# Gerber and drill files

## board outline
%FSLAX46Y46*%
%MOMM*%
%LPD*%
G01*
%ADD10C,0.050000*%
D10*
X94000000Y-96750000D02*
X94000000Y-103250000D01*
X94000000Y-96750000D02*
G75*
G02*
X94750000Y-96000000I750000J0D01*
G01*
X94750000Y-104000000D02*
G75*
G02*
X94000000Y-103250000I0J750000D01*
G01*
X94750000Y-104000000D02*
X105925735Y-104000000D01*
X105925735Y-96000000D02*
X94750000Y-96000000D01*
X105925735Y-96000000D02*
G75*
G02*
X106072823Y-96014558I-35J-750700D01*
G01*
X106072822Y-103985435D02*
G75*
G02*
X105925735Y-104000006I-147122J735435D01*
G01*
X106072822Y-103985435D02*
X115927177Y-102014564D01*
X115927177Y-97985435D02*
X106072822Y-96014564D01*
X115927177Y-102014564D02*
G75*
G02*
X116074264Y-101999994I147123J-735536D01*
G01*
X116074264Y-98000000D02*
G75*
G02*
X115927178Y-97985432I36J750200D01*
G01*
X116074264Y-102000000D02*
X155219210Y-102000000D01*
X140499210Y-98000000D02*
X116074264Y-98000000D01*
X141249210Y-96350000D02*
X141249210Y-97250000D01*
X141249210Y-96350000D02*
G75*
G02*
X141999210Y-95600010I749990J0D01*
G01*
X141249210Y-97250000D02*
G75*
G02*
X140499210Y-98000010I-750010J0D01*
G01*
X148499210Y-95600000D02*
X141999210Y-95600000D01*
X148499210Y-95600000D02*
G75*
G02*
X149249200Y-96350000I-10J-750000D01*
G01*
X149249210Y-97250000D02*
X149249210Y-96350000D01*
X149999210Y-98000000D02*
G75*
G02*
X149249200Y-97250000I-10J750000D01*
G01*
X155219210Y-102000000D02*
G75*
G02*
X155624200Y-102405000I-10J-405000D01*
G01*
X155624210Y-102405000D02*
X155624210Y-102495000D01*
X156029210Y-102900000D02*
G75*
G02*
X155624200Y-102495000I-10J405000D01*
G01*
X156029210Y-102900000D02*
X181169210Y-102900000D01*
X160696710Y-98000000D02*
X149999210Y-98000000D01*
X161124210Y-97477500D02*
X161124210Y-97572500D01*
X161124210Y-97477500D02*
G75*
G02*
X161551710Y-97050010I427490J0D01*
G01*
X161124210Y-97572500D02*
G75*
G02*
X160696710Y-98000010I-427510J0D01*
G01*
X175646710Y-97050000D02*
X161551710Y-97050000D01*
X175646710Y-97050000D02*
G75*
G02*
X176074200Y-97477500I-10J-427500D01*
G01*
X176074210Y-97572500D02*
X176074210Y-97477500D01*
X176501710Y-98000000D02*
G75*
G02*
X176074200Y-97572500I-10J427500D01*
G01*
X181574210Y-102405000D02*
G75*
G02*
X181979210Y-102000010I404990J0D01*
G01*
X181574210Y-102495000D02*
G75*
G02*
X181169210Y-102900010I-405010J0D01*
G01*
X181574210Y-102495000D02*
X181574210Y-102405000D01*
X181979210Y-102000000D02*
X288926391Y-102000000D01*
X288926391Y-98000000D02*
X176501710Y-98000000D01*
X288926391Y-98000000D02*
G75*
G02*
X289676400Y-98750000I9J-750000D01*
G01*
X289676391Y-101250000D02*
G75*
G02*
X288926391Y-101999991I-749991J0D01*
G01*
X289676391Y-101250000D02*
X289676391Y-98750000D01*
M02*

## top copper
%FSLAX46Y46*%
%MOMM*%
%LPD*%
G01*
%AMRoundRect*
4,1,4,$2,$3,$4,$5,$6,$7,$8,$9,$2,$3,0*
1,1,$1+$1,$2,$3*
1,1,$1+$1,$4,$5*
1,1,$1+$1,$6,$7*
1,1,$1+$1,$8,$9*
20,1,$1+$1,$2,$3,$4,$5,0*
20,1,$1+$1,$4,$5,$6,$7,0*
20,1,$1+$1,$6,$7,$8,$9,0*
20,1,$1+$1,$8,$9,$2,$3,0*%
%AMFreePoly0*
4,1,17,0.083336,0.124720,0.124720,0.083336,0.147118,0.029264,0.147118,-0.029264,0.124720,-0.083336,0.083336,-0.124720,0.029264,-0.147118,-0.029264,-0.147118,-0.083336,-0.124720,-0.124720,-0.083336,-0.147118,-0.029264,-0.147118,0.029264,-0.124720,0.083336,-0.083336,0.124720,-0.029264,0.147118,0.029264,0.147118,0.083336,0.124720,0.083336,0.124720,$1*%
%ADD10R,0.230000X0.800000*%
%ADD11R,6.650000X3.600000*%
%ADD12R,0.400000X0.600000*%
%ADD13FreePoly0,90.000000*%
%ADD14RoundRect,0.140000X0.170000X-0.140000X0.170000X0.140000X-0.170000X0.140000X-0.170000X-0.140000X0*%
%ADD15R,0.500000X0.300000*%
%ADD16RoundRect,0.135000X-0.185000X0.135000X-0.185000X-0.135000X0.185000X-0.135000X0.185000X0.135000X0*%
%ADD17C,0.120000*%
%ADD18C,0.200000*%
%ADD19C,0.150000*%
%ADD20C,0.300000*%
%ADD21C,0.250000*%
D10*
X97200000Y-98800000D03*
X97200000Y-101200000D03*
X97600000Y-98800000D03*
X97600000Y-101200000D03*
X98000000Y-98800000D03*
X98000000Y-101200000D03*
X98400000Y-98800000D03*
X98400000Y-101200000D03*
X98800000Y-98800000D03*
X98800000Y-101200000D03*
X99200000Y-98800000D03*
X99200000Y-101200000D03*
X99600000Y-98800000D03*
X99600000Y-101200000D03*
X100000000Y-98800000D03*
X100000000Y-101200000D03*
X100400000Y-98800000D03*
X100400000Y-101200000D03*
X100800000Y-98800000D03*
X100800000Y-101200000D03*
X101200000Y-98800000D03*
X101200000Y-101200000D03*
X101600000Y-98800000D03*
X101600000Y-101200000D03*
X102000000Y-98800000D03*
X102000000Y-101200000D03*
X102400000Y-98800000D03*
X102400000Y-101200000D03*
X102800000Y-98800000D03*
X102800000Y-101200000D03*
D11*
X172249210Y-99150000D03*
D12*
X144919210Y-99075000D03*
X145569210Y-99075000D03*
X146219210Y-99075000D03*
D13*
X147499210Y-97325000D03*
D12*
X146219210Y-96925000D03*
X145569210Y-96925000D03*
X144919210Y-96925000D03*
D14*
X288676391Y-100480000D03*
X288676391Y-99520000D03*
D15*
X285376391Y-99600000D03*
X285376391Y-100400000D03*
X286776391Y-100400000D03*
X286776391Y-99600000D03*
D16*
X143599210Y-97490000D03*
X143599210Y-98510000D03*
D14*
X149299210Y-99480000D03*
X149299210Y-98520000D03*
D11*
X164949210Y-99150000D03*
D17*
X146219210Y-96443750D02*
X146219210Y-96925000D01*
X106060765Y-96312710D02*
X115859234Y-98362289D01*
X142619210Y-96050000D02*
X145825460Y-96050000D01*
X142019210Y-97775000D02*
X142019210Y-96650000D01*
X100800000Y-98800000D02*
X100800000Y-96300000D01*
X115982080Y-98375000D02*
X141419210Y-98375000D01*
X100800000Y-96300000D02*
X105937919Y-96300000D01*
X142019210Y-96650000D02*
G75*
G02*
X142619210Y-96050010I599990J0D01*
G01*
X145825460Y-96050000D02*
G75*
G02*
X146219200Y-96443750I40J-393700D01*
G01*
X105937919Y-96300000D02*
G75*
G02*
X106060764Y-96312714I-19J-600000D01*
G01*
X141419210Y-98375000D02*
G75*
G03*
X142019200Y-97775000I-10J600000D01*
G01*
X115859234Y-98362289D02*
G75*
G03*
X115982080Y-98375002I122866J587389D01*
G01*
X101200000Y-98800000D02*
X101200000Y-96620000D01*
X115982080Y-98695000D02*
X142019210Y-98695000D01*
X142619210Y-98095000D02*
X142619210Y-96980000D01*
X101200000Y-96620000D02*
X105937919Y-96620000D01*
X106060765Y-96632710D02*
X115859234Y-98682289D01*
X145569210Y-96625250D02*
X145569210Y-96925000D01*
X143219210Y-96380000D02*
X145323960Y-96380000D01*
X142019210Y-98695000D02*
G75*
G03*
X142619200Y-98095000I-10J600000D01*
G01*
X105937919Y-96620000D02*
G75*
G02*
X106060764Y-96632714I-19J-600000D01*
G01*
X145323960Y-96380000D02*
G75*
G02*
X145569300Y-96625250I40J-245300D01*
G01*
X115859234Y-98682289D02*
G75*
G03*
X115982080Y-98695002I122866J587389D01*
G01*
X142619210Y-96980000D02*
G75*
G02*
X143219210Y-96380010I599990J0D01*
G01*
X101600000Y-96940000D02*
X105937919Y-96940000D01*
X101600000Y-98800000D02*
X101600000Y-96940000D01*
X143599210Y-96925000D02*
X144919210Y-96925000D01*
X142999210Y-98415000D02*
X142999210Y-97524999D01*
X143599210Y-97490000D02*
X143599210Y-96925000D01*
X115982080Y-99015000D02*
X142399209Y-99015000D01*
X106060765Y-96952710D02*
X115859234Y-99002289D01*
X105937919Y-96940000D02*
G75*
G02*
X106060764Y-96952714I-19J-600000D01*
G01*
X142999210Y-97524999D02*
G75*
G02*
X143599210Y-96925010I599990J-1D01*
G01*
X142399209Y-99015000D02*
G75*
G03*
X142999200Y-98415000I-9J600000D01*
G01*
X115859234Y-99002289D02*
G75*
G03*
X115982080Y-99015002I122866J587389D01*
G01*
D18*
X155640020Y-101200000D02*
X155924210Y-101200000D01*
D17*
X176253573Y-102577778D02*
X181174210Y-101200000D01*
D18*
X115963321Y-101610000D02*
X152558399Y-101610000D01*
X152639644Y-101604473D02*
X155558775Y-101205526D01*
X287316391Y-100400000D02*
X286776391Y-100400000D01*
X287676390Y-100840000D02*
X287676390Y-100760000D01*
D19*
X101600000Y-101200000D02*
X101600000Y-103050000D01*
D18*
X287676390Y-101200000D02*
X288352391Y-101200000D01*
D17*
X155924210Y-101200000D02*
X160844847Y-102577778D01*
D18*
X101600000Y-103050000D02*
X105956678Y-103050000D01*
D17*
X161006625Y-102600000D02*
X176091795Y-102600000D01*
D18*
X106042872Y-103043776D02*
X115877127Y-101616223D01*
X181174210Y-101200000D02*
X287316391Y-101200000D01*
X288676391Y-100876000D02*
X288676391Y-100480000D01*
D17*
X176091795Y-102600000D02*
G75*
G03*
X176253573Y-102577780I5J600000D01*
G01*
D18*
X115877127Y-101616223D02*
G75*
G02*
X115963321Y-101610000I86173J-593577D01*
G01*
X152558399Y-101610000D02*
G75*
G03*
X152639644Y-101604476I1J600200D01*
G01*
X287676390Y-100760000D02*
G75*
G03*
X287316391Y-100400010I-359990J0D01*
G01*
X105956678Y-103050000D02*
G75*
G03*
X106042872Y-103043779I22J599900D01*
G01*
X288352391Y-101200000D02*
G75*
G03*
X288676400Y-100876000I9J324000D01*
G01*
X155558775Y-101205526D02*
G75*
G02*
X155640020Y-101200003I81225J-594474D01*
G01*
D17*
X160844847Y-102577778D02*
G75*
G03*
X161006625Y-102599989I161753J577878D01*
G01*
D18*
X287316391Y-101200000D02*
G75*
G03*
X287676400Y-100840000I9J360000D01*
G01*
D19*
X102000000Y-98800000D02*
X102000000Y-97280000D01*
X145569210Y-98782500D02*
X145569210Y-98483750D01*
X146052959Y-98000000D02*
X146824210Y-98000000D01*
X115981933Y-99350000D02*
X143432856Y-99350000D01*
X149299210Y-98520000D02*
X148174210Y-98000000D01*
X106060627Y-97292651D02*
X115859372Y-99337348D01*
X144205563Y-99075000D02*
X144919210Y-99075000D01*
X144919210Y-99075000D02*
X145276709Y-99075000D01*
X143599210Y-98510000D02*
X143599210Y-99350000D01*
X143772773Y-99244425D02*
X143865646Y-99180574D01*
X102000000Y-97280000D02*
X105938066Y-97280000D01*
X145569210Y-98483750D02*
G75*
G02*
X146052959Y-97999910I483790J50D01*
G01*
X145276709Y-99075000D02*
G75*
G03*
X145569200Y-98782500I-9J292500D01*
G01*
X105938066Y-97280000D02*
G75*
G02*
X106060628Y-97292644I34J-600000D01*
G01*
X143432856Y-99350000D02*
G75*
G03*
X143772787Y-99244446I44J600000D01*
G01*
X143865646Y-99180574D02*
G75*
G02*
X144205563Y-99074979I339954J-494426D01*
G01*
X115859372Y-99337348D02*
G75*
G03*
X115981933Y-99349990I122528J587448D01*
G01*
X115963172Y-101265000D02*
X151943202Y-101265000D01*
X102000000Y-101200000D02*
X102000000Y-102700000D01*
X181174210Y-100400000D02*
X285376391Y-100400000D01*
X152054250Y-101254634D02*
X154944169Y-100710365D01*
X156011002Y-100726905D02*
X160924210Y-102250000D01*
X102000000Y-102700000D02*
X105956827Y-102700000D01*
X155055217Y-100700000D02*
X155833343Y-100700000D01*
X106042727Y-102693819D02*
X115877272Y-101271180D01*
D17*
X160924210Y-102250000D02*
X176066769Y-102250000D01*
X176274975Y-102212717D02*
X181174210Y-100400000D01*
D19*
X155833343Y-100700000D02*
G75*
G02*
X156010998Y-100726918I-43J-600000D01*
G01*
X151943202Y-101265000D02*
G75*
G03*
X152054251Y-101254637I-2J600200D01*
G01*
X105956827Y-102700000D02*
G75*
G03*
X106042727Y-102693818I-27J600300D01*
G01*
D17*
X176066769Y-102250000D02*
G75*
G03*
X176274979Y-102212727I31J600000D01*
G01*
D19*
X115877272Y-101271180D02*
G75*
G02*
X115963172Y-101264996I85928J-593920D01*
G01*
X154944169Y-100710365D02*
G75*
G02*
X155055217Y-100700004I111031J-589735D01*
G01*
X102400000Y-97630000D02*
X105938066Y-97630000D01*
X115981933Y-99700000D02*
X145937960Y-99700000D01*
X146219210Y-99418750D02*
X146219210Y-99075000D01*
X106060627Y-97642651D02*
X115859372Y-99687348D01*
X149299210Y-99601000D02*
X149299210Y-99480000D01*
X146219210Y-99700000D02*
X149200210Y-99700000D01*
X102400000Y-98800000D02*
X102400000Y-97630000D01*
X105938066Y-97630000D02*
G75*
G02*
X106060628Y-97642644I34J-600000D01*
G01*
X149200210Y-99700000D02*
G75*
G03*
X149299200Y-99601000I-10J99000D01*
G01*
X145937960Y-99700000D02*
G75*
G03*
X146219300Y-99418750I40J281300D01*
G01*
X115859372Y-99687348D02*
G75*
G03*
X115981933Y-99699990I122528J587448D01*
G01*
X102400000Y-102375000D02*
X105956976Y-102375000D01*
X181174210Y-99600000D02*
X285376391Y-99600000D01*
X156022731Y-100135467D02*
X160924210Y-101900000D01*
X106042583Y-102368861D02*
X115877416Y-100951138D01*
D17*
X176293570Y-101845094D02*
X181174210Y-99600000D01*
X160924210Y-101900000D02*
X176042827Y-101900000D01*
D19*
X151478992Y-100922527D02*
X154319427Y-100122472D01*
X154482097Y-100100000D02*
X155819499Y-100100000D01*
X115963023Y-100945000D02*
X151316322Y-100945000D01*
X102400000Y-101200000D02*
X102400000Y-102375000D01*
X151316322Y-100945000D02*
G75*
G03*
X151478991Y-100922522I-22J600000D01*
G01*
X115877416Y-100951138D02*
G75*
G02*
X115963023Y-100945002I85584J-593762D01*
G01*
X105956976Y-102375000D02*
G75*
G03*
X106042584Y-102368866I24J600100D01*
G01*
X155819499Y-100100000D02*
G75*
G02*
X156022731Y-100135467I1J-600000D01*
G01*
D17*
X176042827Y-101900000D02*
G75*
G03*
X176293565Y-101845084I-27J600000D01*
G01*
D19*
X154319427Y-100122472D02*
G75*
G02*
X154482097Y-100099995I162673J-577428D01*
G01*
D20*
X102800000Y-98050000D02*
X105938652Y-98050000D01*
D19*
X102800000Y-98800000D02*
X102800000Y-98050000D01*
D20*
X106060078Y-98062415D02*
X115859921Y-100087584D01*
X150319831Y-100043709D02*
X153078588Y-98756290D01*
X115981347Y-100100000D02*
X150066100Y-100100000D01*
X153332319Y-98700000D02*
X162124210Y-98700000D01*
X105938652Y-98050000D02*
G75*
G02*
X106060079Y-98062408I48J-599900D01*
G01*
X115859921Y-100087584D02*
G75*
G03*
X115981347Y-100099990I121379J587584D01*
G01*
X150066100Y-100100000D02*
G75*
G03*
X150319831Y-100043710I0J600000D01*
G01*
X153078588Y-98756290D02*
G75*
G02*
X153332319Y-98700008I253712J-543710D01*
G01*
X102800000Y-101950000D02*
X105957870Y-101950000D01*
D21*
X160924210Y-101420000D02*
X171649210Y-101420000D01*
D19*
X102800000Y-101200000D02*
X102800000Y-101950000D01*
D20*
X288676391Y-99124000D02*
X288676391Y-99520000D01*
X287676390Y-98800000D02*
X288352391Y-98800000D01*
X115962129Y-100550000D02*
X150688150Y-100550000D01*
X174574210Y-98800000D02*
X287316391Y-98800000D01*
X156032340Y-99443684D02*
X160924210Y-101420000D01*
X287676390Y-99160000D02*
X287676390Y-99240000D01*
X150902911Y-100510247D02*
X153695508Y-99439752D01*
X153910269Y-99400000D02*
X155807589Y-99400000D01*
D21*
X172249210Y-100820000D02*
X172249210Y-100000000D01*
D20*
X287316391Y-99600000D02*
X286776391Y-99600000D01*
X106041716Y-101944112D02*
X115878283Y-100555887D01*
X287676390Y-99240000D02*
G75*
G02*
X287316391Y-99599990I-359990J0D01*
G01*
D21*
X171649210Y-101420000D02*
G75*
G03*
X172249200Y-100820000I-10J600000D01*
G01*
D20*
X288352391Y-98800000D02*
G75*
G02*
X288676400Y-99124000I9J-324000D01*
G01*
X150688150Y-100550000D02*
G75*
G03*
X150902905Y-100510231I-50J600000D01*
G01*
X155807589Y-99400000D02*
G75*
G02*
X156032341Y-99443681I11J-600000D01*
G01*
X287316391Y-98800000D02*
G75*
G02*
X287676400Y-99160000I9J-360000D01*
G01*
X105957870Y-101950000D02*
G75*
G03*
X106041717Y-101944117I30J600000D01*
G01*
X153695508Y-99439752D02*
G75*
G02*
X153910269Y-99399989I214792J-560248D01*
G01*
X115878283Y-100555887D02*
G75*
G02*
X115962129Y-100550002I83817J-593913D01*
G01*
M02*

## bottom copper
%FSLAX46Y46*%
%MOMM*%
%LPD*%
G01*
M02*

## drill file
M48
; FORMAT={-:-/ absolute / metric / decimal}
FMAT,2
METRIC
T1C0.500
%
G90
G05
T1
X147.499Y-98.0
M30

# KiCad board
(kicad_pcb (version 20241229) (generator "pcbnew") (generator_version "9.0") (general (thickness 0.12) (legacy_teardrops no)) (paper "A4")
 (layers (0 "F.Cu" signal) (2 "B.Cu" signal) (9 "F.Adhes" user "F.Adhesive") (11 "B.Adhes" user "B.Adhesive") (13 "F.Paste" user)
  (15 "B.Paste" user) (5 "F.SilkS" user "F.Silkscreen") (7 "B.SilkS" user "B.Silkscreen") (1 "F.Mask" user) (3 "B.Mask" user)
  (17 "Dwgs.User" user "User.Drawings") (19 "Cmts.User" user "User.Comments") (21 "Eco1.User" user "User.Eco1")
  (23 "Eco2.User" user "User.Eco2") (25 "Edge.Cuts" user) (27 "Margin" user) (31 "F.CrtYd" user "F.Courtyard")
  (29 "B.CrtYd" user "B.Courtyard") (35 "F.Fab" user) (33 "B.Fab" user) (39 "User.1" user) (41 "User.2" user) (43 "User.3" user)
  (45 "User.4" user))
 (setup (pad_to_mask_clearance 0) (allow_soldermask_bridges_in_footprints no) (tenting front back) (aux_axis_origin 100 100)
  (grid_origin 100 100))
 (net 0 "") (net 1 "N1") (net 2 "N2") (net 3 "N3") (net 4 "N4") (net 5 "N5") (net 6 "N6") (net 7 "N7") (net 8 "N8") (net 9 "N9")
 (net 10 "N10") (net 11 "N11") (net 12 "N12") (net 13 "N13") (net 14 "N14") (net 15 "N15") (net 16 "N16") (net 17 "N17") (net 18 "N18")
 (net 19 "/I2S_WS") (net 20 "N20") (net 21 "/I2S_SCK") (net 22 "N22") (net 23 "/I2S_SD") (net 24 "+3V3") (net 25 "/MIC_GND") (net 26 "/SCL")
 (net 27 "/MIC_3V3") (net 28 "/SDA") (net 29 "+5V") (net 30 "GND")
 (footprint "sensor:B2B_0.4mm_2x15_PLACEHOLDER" (layer "F.Cu") (at 100 100)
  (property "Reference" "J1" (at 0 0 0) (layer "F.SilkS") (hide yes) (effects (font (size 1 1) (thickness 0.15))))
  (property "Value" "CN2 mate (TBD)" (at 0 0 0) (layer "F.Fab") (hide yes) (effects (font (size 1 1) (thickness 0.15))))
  (pad "1" smd rect (at -2.8 -1.2) (size 0.23 0.8) (layers "F.Cu" "F.Mask" "F.Paste") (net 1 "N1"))
  (pad "2" smd rect (at -2.8 1.2) (size 0.23 0.8) (layers "F.Cu" "F.Mask" "F.Paste") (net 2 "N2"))
  (pad "3" smd rect (at -2.4 -1.2) (size 0.23 0.8) (layers "F.Cu" "F.Mask" "F.Paste") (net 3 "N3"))
  (pad "4" smd rect (at -2.4 1.2) (size 0.23 0.8) (layers "F.Cu" "F.Mask" "F.Paste") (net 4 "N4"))
  (pad "5" smd rect (at -2 -1.2) (size 0.23 0.8) (layers "F.Cu" "F.Mask" "F.Paste") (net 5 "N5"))
  (pad "6" smd rect (at -2 1.2) (size 0.23 0.8) (layers "F.Cu" "F.Mask" "F.Paste") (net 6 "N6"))
  (pad "7" smd rect (at -1.6 -1.2) (size 0.23 0.8) (layers "F.Cu" "F.Mask" "F.Paste") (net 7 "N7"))
  (pad "8" smd rect (at -1.6 1.2) (size 0.23 0.8) (layers "F.Cu" "F.Mask" "F.Paste") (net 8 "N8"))
  (pad "9" smd rect (at -1.2 -1.2) (size 0.23 0.8) (layers "F.Cu" "F.Mask" "F.Paste") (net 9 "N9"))
  (pad "10" smd rect (at -1.2 1.2) (size 0.23 0.8) (layers "F.Cu" "F.Mask" "F.Paste") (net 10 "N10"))
  (pad "11" smd rect (at -0.8 -1.2) (size 0.23 0.8) (layers "F.Cu" "F.Mask" "F.Paste") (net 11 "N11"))
  (pad "12" smd rect (at -0.8 1.2) (size 0.23 0.8) (layers "F.Cu" "F.Mask" "F.Paste") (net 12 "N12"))
  (pad "13" smd rect (at -0.4 -1.2) (size 0.23 0.8) (layers "F.Cu" "F.Mask" "F.Paste") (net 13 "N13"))
  (pad "14" smd rect (at -0.4 1.2) (size 0.23 0.8) (layers "F.Cu" "F.Mask" "F.Paste") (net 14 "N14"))
  (pad "15" smd rect (at 0 -1.2) (size 0.23 0.8) (layers "F.Cu" "F.Mask" "F.Paste") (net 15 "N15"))
  (pad "16" smd rect (at 0 1.2) (size 0.23 0.8) (layers "F.Cu" "F.Mask" "F.Paste") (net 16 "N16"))
  (pad "17" smd rect (at 0.4 -1.2) (size 0.23 0.8) (layers "F.Cu" "F.Mask" "F.Paste") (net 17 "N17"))
  (pad "18" smd rect (at 0.4 1.2) (size 0.23 0.8) (layers "F.Cu" "F.Mask" "F.Paste") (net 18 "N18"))
  (pad "19" smd rect (at 0.8 -1.2) (size 0.23 0.8) (layers "F.Cu" "F.Mask" "F.Paste") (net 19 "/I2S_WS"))
  (pad "20" smd rect (at 0.8 1.2) (size 0.23 0.8) (layers "F.Cu" "F.Mask" "F.Paste") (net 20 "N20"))
  (pad "21" smd rect (at 1.2 -1.2) (size 0.23 0.8) (layers "F.Cu" "F.Mask" "F.Paste") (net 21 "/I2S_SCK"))
  (pad "22" smd rect (at 1.2 1.2) (size 0.23 0.8) (layers "F.Cu" "F.Mask" "F.Paste") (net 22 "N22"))
  (pad "23" smd rect (at 1.6 -1.2) (size 0.23 0.8) (layers "F.Cu" "F.Mask" "F.Paste") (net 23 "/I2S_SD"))
  (pad "24" smd rect (at 1.6 1.2) (size 0.23 0.8) (layers "F.Cu" "F.Mask" "F.Paste") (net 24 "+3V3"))
  (pad "25" smd rect (at 2 -1.2) (size 0.23 0.8) (layers "F.Cu" "F.Mask" "F.Paste") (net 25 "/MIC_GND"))
  (pad "26" smd rect (at 2 1.2) (size 0.23 0.8) (layers "F.Cu" "F.Mask" "F.Paste") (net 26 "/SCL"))
  (pad "27" smd rect (at 2.4 -1.2) (size 0.23 0.8) (layers "F.Cu" "F.Mask" "F.Paste") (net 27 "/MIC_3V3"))
  (pad "28" smd rect (at 2.4 1.2) (size 0.23 0.8) (layers "F.Cu" "F.Mask" "F.Paste") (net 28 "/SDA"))
  (pad "29" smd rect (at 2.8 -1.2) (size 0.23 0.8) (layers "F.Cu" "F.Mask" "F.Paste") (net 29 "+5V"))
  (pad "30" smd rect (at 2.8 1.2) (size 0.23 0.8) (layers "F.Cu" "F.Mask" "F.Paste") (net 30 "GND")))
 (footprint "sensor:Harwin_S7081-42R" (layer "F.Cu") (at 172.24921 99.15)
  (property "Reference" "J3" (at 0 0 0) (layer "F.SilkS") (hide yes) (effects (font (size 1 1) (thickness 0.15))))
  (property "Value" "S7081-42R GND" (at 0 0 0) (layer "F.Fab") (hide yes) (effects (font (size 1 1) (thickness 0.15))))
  (pad "1" smd rect (at 0 0) (size 6.65 3.6) (layers "F.Cu" "F.Mask" "F.Paste") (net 30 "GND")))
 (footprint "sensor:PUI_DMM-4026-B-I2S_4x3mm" (layer "F.Cu") (at 146.49921 98 90)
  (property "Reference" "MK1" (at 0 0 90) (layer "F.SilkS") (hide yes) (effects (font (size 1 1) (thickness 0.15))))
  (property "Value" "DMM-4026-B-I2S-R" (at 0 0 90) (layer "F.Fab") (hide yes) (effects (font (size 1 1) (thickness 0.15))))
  (pad "" np_thru_hole circle (at 0 1 90) (size 0.5 0.5) (drill 0.5) (layers "*.Mask"))
  (pad "1" smd rect (at -1.075 -1.58 90) (size 0.6 0.4) (layers "F.Cu" "F.Mask" "F.Paste") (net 25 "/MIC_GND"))
  (pad "2" smd rect (at -1.075 -0.93 90) (size 0.6 0.4) (layers "F.Cu" "F.Mask" "F.Paste") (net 25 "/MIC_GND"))
  (pad "3" smd rect (at -1.075 -0.28 90) (size 0.6 0.4) (layers "F.Cu" "F.Mask" "F.Paste") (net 27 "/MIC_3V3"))
  (pad "4" smd custom (at 0.675 1 90) (size 0.3 0.3) (layers "F.Cu" "F.Mask" "F.Paste") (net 25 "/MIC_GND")
   (options (clearance outline) (anchor circle)) (primitives))
  (pad "5" smd rect (at 1.075 -0.28 90) (size 0.6 0.4) (layers "F.Cu" "F.Mask" "F.Paste") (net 19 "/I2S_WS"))
  (pad "6" smd rect (at 1.075 -0.93 90) (size 0.6 0.4) (layers "F.Cu" "F.Mask" "F.Paste") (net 21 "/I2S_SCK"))
  (pad "7" smd rect (at 1.075 -1.58 90) (size 0.6 0.4) (layers "F.Cu" "F.Mask" "F.Paste") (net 23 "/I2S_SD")))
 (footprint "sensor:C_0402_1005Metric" (layer "F.Cu") (at 288.676391 100 90)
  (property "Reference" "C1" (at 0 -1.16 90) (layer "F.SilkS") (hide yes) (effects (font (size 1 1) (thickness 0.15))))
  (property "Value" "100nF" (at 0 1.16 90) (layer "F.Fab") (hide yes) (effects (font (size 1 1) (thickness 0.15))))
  (pad "1" smd roundrect (at -0.48 0 90) (size 0.56 0.62) (layers "F.Cu" "F.Mask" "F.Paste") (roundrect_rratio 0.25) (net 24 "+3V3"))
  (pad "2" smd roundrect (at 0.48 0 90) (size 0.56 0.62) (layers "F.Cu" "F.Mask" "F.Paste") (roundrect_rratio 0.25) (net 30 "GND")))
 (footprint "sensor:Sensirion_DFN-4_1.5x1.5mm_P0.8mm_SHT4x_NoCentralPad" (layer "F.Cu") (at 286.076391 100)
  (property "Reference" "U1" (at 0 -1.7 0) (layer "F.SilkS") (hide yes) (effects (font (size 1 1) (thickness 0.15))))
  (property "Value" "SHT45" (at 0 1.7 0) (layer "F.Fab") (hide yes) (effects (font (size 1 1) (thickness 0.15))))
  (pad "1" smd rect (at -0.7 -0.4) (size 0.5 0.3) (layers "F.Cu" "F.Mask" "F.Paste") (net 28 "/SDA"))
  (pad "2" smd rect (at -0.7 0.4) (size 0.5 0.3) (layers "F.Cu" "F.Mask" "F.Paste") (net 26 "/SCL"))
  (pad "3" smd rect (at 0.7 0.4) (size 0.5 0.3) (layers "F.Cu" "F.Mask" "F.Paste") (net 24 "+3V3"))
  (pad "4" smd rect (at 0.7 -0.4) (size 0.5 0.3) (layers "F.Cu" "F.Mask" "F.Paste") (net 30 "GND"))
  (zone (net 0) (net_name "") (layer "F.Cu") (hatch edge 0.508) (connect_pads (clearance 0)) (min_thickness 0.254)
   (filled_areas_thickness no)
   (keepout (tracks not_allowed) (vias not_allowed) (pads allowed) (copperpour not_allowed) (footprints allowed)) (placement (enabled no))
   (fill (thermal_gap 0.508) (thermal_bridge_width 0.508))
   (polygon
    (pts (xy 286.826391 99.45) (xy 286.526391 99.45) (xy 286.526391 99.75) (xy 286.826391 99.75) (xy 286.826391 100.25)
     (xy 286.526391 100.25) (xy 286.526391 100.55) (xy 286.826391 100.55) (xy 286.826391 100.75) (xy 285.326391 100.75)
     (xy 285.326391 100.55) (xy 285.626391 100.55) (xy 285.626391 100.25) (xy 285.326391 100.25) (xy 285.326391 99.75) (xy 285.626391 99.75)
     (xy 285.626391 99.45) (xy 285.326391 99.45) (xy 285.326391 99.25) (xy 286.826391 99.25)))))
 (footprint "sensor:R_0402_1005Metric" (layer "F.Cu") (at 143.59921 98 -90)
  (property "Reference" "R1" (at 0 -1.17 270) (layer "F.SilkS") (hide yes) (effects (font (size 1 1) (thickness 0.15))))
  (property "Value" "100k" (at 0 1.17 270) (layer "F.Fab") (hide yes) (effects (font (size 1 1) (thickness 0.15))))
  (pad "1" smd roundrect (at -0.51 0 270) (size 0.54 0.64) (layers "F.Cu" "F.Mask" "F.Paste") (roundrect_rratio 0.25) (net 23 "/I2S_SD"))
  (pad "2" smd roundrect (at 0.51 0 270) (size 0.54 0.64) (layers "F.Cu" "F.Mask" "F.Paste") (roundrect_rratio 0.25) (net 25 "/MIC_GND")))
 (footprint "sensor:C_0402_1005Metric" (layer "F.Cu") (at 149.29921 99 90)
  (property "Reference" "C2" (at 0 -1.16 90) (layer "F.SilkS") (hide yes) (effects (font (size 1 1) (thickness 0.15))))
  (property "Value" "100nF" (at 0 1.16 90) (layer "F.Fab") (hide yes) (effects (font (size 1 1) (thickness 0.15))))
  (pad "1" smd roundrect (at -0.48 0 90) (size 0.56 0.62) (layers "F.Cu" "F.Mask" "F.Paste") (roundrect_rratio 0.25) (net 27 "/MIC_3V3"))
  (pad "2" smd roundrect (at 0.48 0 90) (size 0.56 0.62) (layers "F.Cu" "F.Mask" "F.Paste") (roundrect_rratio 0.25) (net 25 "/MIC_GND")))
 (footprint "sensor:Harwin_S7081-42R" (layer "F.Cu") (at 164.94921 99.15)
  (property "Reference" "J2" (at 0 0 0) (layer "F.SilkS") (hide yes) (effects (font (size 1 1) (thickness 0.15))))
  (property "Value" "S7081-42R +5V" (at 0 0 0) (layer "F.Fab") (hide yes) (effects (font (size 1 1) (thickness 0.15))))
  (pad "1" smd rect (at 0 0) (size 6.65 3.6) (layers "F.Cu" "F.Mask" "F.Paste") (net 29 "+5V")))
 (gr_line (start 94 96.75) (end 94 103.25) (stroke (width 0.05) (type default)) (layer "Edge.Cuts"))
 (gr_arc (start 94 96.75) (mid 94.21967 96.21967) (end 94.75 96) (stroke (width 0.05) (type default)) (layer "Edge.Cuts"))
 (gr_arc (start 94.75 104) (mid 94.21967 103.78033) (end 94 103.25) (stroke (width 0.05) (type default)) (layer "Edge.Cuts"))
 (gr_line (start 94.75 104) (end 105.925735 104) (stroke (width 0.05) (type default)) (layer "Edge.Cuts"))
 (gr_line (start 105.925735 96) (end 94.75 96) (stroke (width 0.05) (type default)) (layer "Edge.Cuts"))
 (gr_arc (start 105.925735 96) (mid 105.999638 96.003653) (end 106.072822 96.014564) (stroke (width 0.05) (type default))
  (layer "Edge.Cuts"))
 (gr_arc (start 106.072822 103.985435) (mid 105.999638 103.99635) (end 105.925735 104) (stroke (width 0.05) (type default))
  (layer "Edge.Cuts"))
 (gr_line (start 106.072822 103.985435) (end 115.927177 102.014564) (stroke (width 0.05) (type default)) (layer "Edge.Cuts"))
 (gr_line (start 115.927177 97.985435) (end 106.072822 96.014564) (stroke (width 0.05) (type default)) (layer "Edge.Cuts"))
 (gr_arc (start 115.927177 102.014564) (mid 116.000361 102.00365) (end 116.074264 102) (stroke (width 0.05) (type default))
  (layer "Edge.Cuts"))
 (gr_arc (start 116.074264 98) (mid 116.000361 97.996349) (end 115.927177 97.985435) (stroke (width 0.05) (type default))
  (layer "Edge.Cuts"))
 (gr_line (start 116.074264 102) (end 155.21921 102) (stroke (width 0.05) (type default)) (layer "Edge.Cuts"))
 (gr_line (start 140.49921 98) (end 116.074264 98) (stroke (width 0.05) (type default)) (layer "Edge.Cuts"))
 (gr_line (start 141.24921 96.35) (end 141.24921 97.25) (stroke (width 0.05) (type default)) (layer "Edge.Cuts"))
 (gr_arc (start 141.24921 96.35) (mid 141.468881 95.819673) (end 141.99921 95.6) (stroke (width 0.05) (type default)) (layer "Edge.Cuts"))
 (gr_arc (start 141.24921 97.25) (mid 141.02954 97.78033) (end 140.49921 98) (stroke (width 0.05) (type default)) (layer "Edge.Cuts"))
 (gr_line (start 148.49921 95.6) (end 141.99921 95.6) (stroke (width 0.05) (type default)) (layer "Edge.Cuts"))
 (gr_arc (start 148.49921 95.6) (mid 149.029534 95.819673) (end 149.24921 96.35) (stroke (width 0.05) (type default)) (layer "Edge.Cuts"))
 (gr_line (start 149.24921 97.25) (end 149.24921 96.35) (stroke (width 0.05) (type default)) (layer "Edge.Cuts"))
 (gr_arc (start 149.99921 98) (mid 149.46888 97.78033) (end 149.24921 97.25) (stroke (width 0.05) (type default)) (layer "Edge.Cuts"))
 (gr_arc (start 155.21921 102) (mid 155.505588 102.118621) (end 155.62421 102.405) (stroke (width 0.05) (type default)) (layer "Edge.Cuts"))
 (gr_line (start 155.62421 102.405) (end 155.62421 102.495) (stroke (width 0.05) (type default)) (layer "Edge.Cuts"))
 (gr_arc (start 156.02921 102.9) (mid 155.742825 102.781382) (end 155.62421 102.495) (stroke (width 0.05) (type default))
  (layer "Edge.Cuts"))
 (gr_line (start 156.02921 102.9) (end 181.16921 102.9) (stroke (width 0.05) (type default)) (layer "Edge.Cuts"))
 (gr_line (start 160.69671 98) (end 149.99921 98) (stroke (width 0.05) (type default)) (layer "Edge.Cuts"))
 (gr_line (start 161.12421 97.4775) (end 161.12421 97.5725) (stroke (width 0.05) (type default)) (layer "Edge.Cuts"))
 (gr_arc (start 161.12421 97.4775) (mid 161.249422 97.175215) (end 161.55171 97.05) (stroke (width 0.05) (type default)) (layer "Edge.Cuts"))
 (gr_arc (start 161.12421 97.5725) (mid 160.998998 97.874788) (end 160.69671 98) (stroke (width 0.05) (type default)) (layer "Edge.Cuts"))
 (gr_line (start 175.64671 97.05) (end 161.55171 97.05) (stroke (width 0.05) (type default)) (layer "Edge.Cuts"))
 (gr_arc (start 175.64671 97.05) (mid 175.948992 97.175215) (end 176.07421 97.4775) (stroke (width 0.05) (type default)) (layer "Edge.Cuts"))
 (gr_line (start 176.07421 97.5725) (end 176.07421 97.4775) (stroke (width 0.05) (type default)) (layer "Edge.Cuts"))
 (gr_arc (start 176.50171 98) (mid 176.199422 97.874788) (end 176.07421 97.5725) (stroke (width 0.05) (type default)) (layer "Edge.Cuts"))
 (gr_arc (start 181.57421 102.405) (mid 181.692832 102.118621) (end 181.97921 102) (stroke (width 0.05) (type default)) (layer "Edge.Cuts"))
 (gr_arc (start 181.57421 102.495) (mid 181.455589 102.781382) (end 181.16921 102.9) (stroke (width 0.05) (type default))
  (layer "Edge.Cuts"))
 (gr_line (start 181.57421 102.495) (end 181.57421 102.405) (stroke (width 0.05) (type default)) (layer "Edge.Cuts"))
 (gr_line (start 181.97921 102) (end 288.926391 102) (stroke (width 0.05) (type default)) (layer "Edge.Cuts"))
 (gr_line (start 288.926391 98) (end 176.50171 98) (stroke (width 0.05) (type default)) (layer "Edge.Cuts"))
 (gr_arc (start 288.926391 98) (mid 289.456727 98.219667) (end 289.676391 98.75) (stroke (width 0.05) (type default)) (layer "Edge.Cuts"))
 (gr_arc (start 289.676391 101.25) (mid 289.456721 101.780327) (end 288.926391 102) (stroke (width 0.05) (type default)) (layer "Edge.Cuts"))
 (gr_line (start 289.676391 101.25) (end 289.676391 98.75) (stroke (width 0.05) (type default)) (layer "Edge.Cuts"))
 (segment (start 146.21921 96.44375) (end 146.21921 96.925) (width 0.12) (layer "F.Cu") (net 19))
 (segment (start 106.060765 96.31271) (end 115.859234 98.362289) (width 0.12) (layer "F.Cu") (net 19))
 (segment (start 142.61921 96.05) (end 145.82546 96.05) (width 0.12) (layer "F.Cu") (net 19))
 (segment (start 142.01921 97.775) (end 142.01921 96.65) (width 0.12) (layer "F.Cu") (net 19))
 (segment (start 100.8 98.8) (end 100.8 96.3) (width 0.12) (layer "F.Cu") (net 19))
 (segment (start 115.98208 98.375) (end 141.41921 98.375) (width 0.12) (layer "F.Cu") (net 19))
 (segment (start 100.8 96.3) (end 105.937919 96.3) (width 0.12) (layer "F.Cu") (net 19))
 (arc (start 142.01921 96.65) (mid 142.194945 96.225735) (end 142.61921 96.05) (width 0.12) (layer "F.Cu") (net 19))
 (arc (start 145.82546 96.05) (mid 146.103883 96.165326) (end 146.21921 96.44375) (width 0.12) (layer "F.Cu") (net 19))
 (arc (start 105.937919 96.3) (mid 105.99967 96.303186) (end 106.060765 96.31271) (width 0.12) (layer "F.Cu") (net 19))
 (arc (start 141.41921 98.375) (mid 141.843474 98.199264) (end 142.01921 97.775) (width 0.12) (layer "F.Cu") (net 19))
 (arc (start 115.859234 98.362289) (mid 115.920329 98.371813) (end 115.98208 98.375) (width 0.12) (layer "F.Cu") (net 19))
 (segment (start 101.2 98.8) (end 101.2 96.62) (width 0.12) (layer "F.Cu") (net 21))
 (segment (start 115.98208 98.695) (end 142.01921 98.695) (width 0.12) (layer "F.Cu") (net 21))
 (segment (start 142.61921 98.095) (end 142.61921 96.98) (width 0.12) (layer "F.Cu") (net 21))
 (segment (start 101.2 96.62) (end 105.937919 96.62) (width 0.12) (layer "F.Cu") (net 21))
 (segment (start 106.060765 96.63271) (end 115.859234 98.682289) (width 0.12) (layer "F.Cu") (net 21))
 (segment (start 145.56921 96.62525) (end 145.56921 96.925) (width 0.12) (layer "F.Cu") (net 21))
 (segment (start 143.21921 96.38) (end 145.32396 96.38) (width 0.12) (layer "F.Cu") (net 21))
 (arc (start 142.01921 98.695) (mid 142.443474 98.519264) (end 142.61921 98.095) (width 0.12) (layer "F.Cu") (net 21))
 (arc (start 105.937919 96.62) (mid 105.99967 96.623186) (end 106.060765 96.63271) (width 0.12) (layer "F.Cu") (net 21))
 (arc (start 145.32396 96.38) (mid 145.497377 96.451832) (end 145.56921 96.62525) (width 0.12) (layer "F.Cu") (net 21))
 (arc (start 115.859234 98.682289) (mid 115.920329 98.691813) (end 115.98208 98.695) (width 0.12) (layer "F.Cu") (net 21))
 (arc (start 142.61921 96.98) (mid 142.794945 96.555735) (end 143.21921 96.38) (width 0.12) (layer "F.Cu") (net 21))
 (segment (start 101.6 96.94) (end 105.937919 96.94) (width 0.12) (layer "F.Cu") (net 23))
 (segment (start 101.6 98.8) (end 101.6 96.94) (width 0.12) (layer "F.Cu") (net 23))
 (segment (start 143.59921 96.925) (end 144.91921 96.925) (width 0.12) (layer "F.Cu") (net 23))
 (segment (start 142.99921 98.415) (end 142.99921 97.524999) (width 0.12) (layer "F.Cu") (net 23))
 (segment (start 143.59921 97.49) (end 143.59921 96.925) (width 0.12) (layer "F.Cu") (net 23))
 (segment (start 115.98208 99.015) (end 142.399209 99.015) (width 0.12) (layer "F.Cu") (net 23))
 (segment (start 106.060765 96.95271) (end 115.859234 99.002289) (width 0.12) (layer "F.Cu") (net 23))
 (arc (start 105.937919 96.94) (mid 105.99967 96.943186) (end 106.060765 96.95271) (width 0.12) (layer "F.Cu") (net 23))
 (arc (start 142.99921 97.524999) (mid 143.174945 97.100735) (end 143.59921 96.925) (width 0.12) (layer "F.Cu") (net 23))
 (arc (start 142.399209 99.015) (mid 142.823474 98.839264) (end 142.99921 98.415) (width 0.12) (layer "F.Cu") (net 23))
 (arc (start 115.859234 99.002289) (mid 115.920329 99.011813) (end 115.98208 99.015) (width 0.12) (layer "F.Cu") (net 23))
 (segment (start 155.64002 101.2) (end 155.92421 101.2) (width 0.2) (layer "F.Cu") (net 24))
 (segment (start 176.253573 102.577778) (end 181.17421 101.2) (width 0.12) (layer "F.Cu") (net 24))
 (segment (start 115.963321 101.61) (end 152.558399 101.61) (width 0.2) (layer "F.Cu") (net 24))
 (segment (start 152.639644 101.604473) (end 155.558775 101.205526) (width 0.2) (layer "F.Cu") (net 24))
 (segment (start 287.316391 100.4) (end 286.776391 100.4) (width 0.2) (layer "F.Cu") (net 24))
 (segment (start 287.67639 100.84) (end 287.67639 100.76) (width 0.2) (layer "F.Cu") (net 24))
 (segment (start 101.6 101.2) (end 101.6 103.05) (width 0.15) (layer "F.Cu") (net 24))
 (segment (start 287.67639 101.2) (end 288.352391 101.2) (width 0.2) (layer "F.Cu") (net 24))
 (segment (start 155.92421 101.2) (end 160.844847 102.577778) (width 0.12) (layer "F.Cu") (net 24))
 (segment (start 101.6 103.05) (end 105.956678 103.05) (width 0.2) (layer "F.Cu") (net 24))
 (segment (start 161.006625 102.6) (end 176.091795 102.6) (width 0.12) (layer "F.Cu") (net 24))
 (segment (start 106.042872 103.043776) (end 115.877127 101.616223) (width 0.2) (layer "F.Cu") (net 24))
 (segment (start 181.17421 101.2) (end 287.316391 101.2) (width 0.2) (layer "F.Cu") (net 24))
 (segment (start 288.676391 100.876) (end 288.676391 100.48) (width 0.2) (layer "F.Cu") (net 24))
 (arc (start 176.091795 102.6) (mid 176.173444 102.594418) (end 176.253573 102.577778) (width 0.12) (layer "F.Cu") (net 24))
 (arc (start 115.877127 101.616223) (mid 115.920112 101.611557) (end 115.963321 101.61) (width 0.2) (layer "F.Cu") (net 24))
 (arc (start 152.558399 101.61) (mid 152.599115 101.608616) (end 152.639644 101.604473) (width 0.2) (layer "F.Cu") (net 24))
 (arc (start 287.67639 100.76) (mid 287.570949 100.505441) (end 287.316391 100.4) (width 0.2) (layer "F.Cu") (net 24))
 (arc (start 105.956678 103.05) (mid 105.999887 103.048442) (end 106.042872 103.043776) (width 0.2) (layer "F.Cu") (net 24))
 (arc (start 288.352391 101.2) (mid 288.581493 101.105102) (end 288.676391 100.876) (width 0.2) (layer "F.Cu") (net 24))
 (arc (start 155.558775 101.205526) (mid 155.599304 101.201383) (end 155.64002 101.2) (width 0.2) (layer "F.Cu") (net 24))
 (arc (start 160.844847 102.577778) (mid 160.924977 102.594418) (end 161.006625 102.6) (width 0.12) (layer "F.Cu") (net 24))
 (arc (start 287.316391 101.2) (mid 287.570949 101.094558) (end 287.67639 100.84) (width 0.2) (layer "F.Cu") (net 24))
 (segment (start 102 98.8) (end 102 97.28) (width 0.15) (layer "F.Cu") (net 25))
 (segment (start 145.56921 98.7825) (end 145.56921 98.48375) (width 0.15) (layer "F.Cu") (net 25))
 (segment (start 146.052959 98) (end 146.82421 98) (width 0.15) (layer "F.Cu") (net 25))
 (segment (start 115.981933 99.35) (end 143.432856 99.35) (width 0.15) (layer "F.Cu") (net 25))
 (segment (start 149.29921 98.52) (end 148.17421 98) (width 0.15) (layer "F.Cu") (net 25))
 (segment (start 106.060627 97.292651) (end 115.859372 99.337348) (width 0.15) (layer "F.Cu") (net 25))
 (segment (start 144.205563 99.075) (end 144.91921 99.075) (width 0.15) (layer "F.Cu") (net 25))
 (segment (start 144.91921 99.075) (end 145.276709 99.075) (width 0.15) (layer "F.Cu") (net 25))
 (segment (start 143.59921 98.51) (end 143.59921 99.35) (width 0.15) (layer "F.Cu") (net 25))
 (segment (start 143.772773 99.244425) (end 143.865646 99.180574) (width 0.15) (layer "F.Cu") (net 25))
 (segment (start 102 97.28) (end 105.938066 97.28) (width 0.15) (layer "F.Cu") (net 25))
 (arc (start 145.56921 98.48375) (mid 145.710897 98.141687) (end 146.052959 98) (width 0.15) (layer "F.Cu") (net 25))
 (arc (start 145.276709 99.075) (mid 145.483538 98.989328) (end 145.56921 98.7825) (width 0.15) (layer "F.Cu") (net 25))
 (arc (start 105.938066 97.28) (mid 105.999672 97.283171) (end 106.060627 97.292651) (width 0.15) (layer "F.Cu") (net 25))
 (arc (start 143.432856 99.35) (mid 143.610823 99.322998) (end 143.772773 99.244425) (width 0.15) (layer "F.Cu") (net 25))
 (arc (start 143.865646 99.180574) (mid 144.027596 99.102001) (end 144.205563 99.075) (width 0.15) (layer "F.Cu") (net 25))
 (arc (start 115.859372 99.337348) (mid 115.920327 99.346828) (end 115.981933 99.35) (width 0.15) (layer "F.Cu") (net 25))
 (segment (start 115.963172 101.265) (end 151.943202 101.265) (width 0.15) (layer "F.Cu") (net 26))
 (segment (start 102 101.2) (end 102 102.7) (width 0.15) (layer "F.Cu") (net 26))
 (segment (start 181.17421 100.4) (end 285.376391 100.4) (width 0.15) (layer "F.Cu") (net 26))
 (segment (start 152.05425 101.254634) (end 154.944169 100.710365) (width 0.15) (layer "F.Cu") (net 26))
 (segment (start 156.011002 100.726905) (end 160.92421 102.25) (width 0.15) (layer "F.Cu") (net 26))
 (segment (start 102 102.7) (end 105.956827 102.7) (width 0.15) (layer "F.Cu") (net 26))
 (segment (start 155.055217 100.7) (end 155.833343 100.7) (width 0.15) (layer "F.Cu") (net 26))
 (segment (start 106.042727 102.693819) (end 115.877272 101.27118) (width 0.15) (layer "F.Cu") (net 26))
 (segment (start 160.92421 102.25) (end 176.066769 102.25) (width 0.12) (layer "F.Cu") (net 26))
 (segment (start 176.274975 102.212717) (end 181.17421 100.4) (width 0.12) (layer "F.Cu") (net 26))
 (arc (start 155.833343 100.7) (mid 155.923186 100.706764) (end 156.011002 100.726905) (width 0.15) (layer "F.Cu") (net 26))
 (arc (start 151.943202 101.265) (mid 151.998967 101.262402) (end 152.05425 101.254634) (width 0.15) (layer "F.Cu") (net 26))
 (arc (start 105.956827 102.7) (mid 105.999888 102.698452) (end 106.042727 102.693819) (width 0.15) (layer "F.Cu") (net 26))
 (arc (start 176.066769 102.25) (mid 176.172528 102.240605) (end 176.274975 102.212717) (width 0.12) (layer "F.Cu") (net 26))
 (arc (start 115.877272 101.27118) (mid 115.920111 101.266547) (end 115.963172 101.265) (width 0.15) (layer "F.Cu") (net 26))
 (arc (start 154.944169 100.710365) (mid 154.999452 100.702597) (end 155.055217 100.7) (width 0.15) (layer "F.Cu") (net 26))
 (segment (start 102.4 97.63) (end 105.938066 97.63) (width 0.15) (layer "F.Cu") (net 27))
 (segment (start 115.981933 99.7) (end 145.93796 99.7) (width 0.15) (layer "F.Cu") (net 27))
 (segment (start 146.21921 99.41875) (end 146.21921 99.075) (width 0.15) (layer "F.Cu") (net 27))
 (segment (start 106.060627 97.642651) (end 115.859372 99.687348) (width 0.15) (layer "F.Cu") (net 27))
 (segment (start 149.29921 99.601) (end 149.29921 99.48) (width 0.15) (layer "F.Cu") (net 27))
 (segment (start 146.21921 99.7) (end 149.20021 99.7) (width 0.15) (layer "F.Cu") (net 27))
 (segment (start 102.4 98.8) (end 102.4 97.63) (width 0.15) (layer "F.Cu") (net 27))
 (arc (start 105.938066 97.63) (mid 105.999672 97.633171) (end 106.060627 97.642651) (width 0.15) (layer "F.Cu") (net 27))
 (arc (start 149.20021 99.7) (mid 149.270213 99.671003) (end 149.29921 99.601) (width 0.15) (layer "F.Cu") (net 27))
 (arc (start 145.93796 99.7) (mid 146.136833 99.617623) (end 146.21921 99.41875) (width 0.15) (layer "F.Cu") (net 27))
 (arc (start 115.859372 99.687348) (mid 115.920327 99.696828) (end 115.981933 99.7) (width 0.15) (layer "F.Cu") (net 27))
 (segment (start 102.4 102.375) (end 105.956976 102.375) (width 0.15) (layer "F.Cu") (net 28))
 (segment (start 181.17421 99.6) (end 285.376391 99.6) (width 0.15) (layer "F.Cu") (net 28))
 (segment (start 156.022731 100.135467) (end 160.92421 101.9) (width 0.15) (layer "F.Cu") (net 28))
 (segment (start 106.042583 102.368861) (end 115.877416 100.951138) (width 0.15) (layer "F.Cu") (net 28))
 (segment (start 176.29357 101.845094) (end 181.17421 99.6) (width 0.12) (layer "F.Cu") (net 28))
 (segment (start 160.92421 101.9) (end 176.042827 101.9) (width 0.12) (layer "F.Cu") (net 28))
 (segment (start 151.478992 100.922527) (end 154.319427 100.122472) (width 0.15) (layer "F.Cu") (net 28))
 (segment (start 154.482097 100.1) (end 155.819499 100.1) (width 0.15) (layer "F.Cu") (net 28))
 (segment (start 115.963023 100.945) (end 151.316322 100.945) (width 0.15) (layer "F.Cu") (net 28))
 (segment (start 102.4 101.2) (end 102.4 102.375) (width 0.15) (layer "F.Cu") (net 28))
 (arc (start 151.316322 100.945) (mid 151.39843 100.939355) (end 151.478992 100.922527) (width 0.15) (layer "F.Cu") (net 28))
 (arc (start 115.877416 100.951138) (mid 115.92011 100.946536) (end 115.963023 100.945) (width 0.15) (layer "F.Cu") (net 28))
 (arc (start 105.956976 102.375) (mid 105.999889 102.373463) (end 106.042583 102.368861) (width 0.15) (layer "F.Cu") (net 28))
 (arc (start 155.819499 100.1) (mid 155.922651 100.108933) (end 156.022731 100.135467) (width 0.15) (layer "F.Cu") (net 28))
 (arc (start 176.042827 101.9) (mid 176.171169 101.886112) (end 176.29357 101.845094) (width 0.12) (layer "F.Cu") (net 28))
 (arc (start 154.319427 100.122472) (mid 154.399989 100.105644) (end 154.482097 100.1) (width 0.15) (layer "F.Cu") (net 28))
 (segment (start 102.8 98.05) (end 105.938652 98.05) (width 0.3) (layer "F.Cu") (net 29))
 (segment (start 102.8 98.8) (end 102.8 98.05) (width 0.15) (layer "F.Cu") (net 29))
 (segment (start 106.060078 98.062415) (end 115.859921 100.087584) (width 0.3) (layer "F.Cu") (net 29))
 (segment (start 150.319831 100.043709) (end 153.078588 98.75629) (width 0.3) (layer "F.Cu") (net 29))
 (segment (start 115.981347 100.1) (end 150.0661 100.1) (width 0.3) (layer "F.Cu") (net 29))
 (segment (start 153.332319 98.7) (end 162.12421 98.7) (width 0.3) (layer "F.Cu") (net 29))
 (arc (start 105.938652 98.05) (mid 105.999681 98.053111) (end 106.060078 98.062415) (width 0.3) (layer "F.Cu") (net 29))
 (arc (start 115.859921 100.087584) (mid 115.920318 100.096888) (end 115.981347 100.1) (width 0.3) (layer "F.Cu") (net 29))
 (arc (start 150.0661 100.1) (mid 150.19605 100.085758) (end 150.319831 100.043709) (width 0.3) (layer "F.Cu") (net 29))
 (arc (start 153.078588 98.75629) (mid 153.202369 98.714241) (end 153.332319 98.7) (width 0.3) (layer "F.Cu") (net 29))
 (segment (start 102.8 101.95) (end 105.95787 101.95) (width 0.3) (layer "F.Cu") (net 30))
 (segment (start 160.92421 101.42) (end 171.64921 101.42) (width 0.25) (layer "F.Cu") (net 30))
 (segment (start 102.8 101.2) (end 102.8 101.95) (width 0.15) (layer "F.Cu") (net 30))
 (segment (start 288.676391 99.124) (end 288.676391 99.52) (width 0.3) (layer "F.Cu") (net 30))
 (segment (start 287.67639 98.8) (end 288.352391 98.8) (width 0.3) (layer "F.Cu") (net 30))
 (segment (start 115.962129 100.55) (end 150.68815 100.55) (width 0.3) (layer "F.Cu") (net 30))
 (segment (start 174.57421 98.8) (end 287.316391 98.8) (width 0.3) (layer "F.Cu") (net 30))
 (segment (start 156.03234 99.443684) (end 160.92421 101.42) (width 0.3) (layer "F.Cu") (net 30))
 (segment (start 287.67639 99.16) (end 287.67639 99.24) (width 0.3) (layer "F.Cu") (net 30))
 (segment (start 150.902911 100.510247) (end 153.695508 99.439752) (width 0.3) (layer "F.Cu") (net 30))
 (segment (start 153.910269 99.4) (end 155.807589 99.4) (width 0.3) (layer "F.Cu") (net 30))
 (segment (start 172.24921 100.82) (end 172.24921 100) (width 0.25) (layer "F.Cu") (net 30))
 (segment (start 287.316391 99.6) (end 286.776391 99.6) (width 0.3) (layer "F.Cu") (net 30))
 (segment (start 106.041716 101.944112) (end 115.878283 100.555887) (width 0.3) (layer "F.Cu") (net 30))
 (arc (start 287.67639 99.24) (mid 287.570949 99.494558) (end 287.316391 99.6) (width 0.3) (layer "F.Cu") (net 30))
 (arc (start 171.64921 101.42) (mid 172.073474 101.244264) (end 172.24921 100.82) (width 0.25) (layer "F.Cu") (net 30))
 (arc (start 288.352391 98.8) (mid 288.581493 98.894897) (end 288.676391 99.124) (width 0.3) (layer "F.Cu") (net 30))
 (arc (start 150.68815 100.55) (mid 150.797354 100.539978) (end 150.902911 100.510247) (width 0.3) (layer "F.Cu") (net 30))
 (arc (start 155.807589 99.4) (mid 155.922068 99.411022) (end 156.03234 99.443684) (width 0.3) (layer "F.Cu") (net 30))
 (arc (start 287.316391 98.8) (mid 287.570949 98.905441) (end 287.67639 99.16) (width 0.3) (layer "F.Cu") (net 30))
 (arc (start 105.95787 101.95) (mid 105.999896 101.948526) (end 106.041716 101.944112) (width 0.3) (layer "F.Cu") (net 30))
 (arc (start 153.695508 99.439752) (mid 153.801065 99.410021) (end 153.910269 99.4) (width 0.3) (layer "F.Cu") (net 30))
 (arc (start 115.878283 100.555887) (mid 115.920103 100.551473) (end 115.962129 100.55) (width 0.3) (layer "F.Cu") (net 30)))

